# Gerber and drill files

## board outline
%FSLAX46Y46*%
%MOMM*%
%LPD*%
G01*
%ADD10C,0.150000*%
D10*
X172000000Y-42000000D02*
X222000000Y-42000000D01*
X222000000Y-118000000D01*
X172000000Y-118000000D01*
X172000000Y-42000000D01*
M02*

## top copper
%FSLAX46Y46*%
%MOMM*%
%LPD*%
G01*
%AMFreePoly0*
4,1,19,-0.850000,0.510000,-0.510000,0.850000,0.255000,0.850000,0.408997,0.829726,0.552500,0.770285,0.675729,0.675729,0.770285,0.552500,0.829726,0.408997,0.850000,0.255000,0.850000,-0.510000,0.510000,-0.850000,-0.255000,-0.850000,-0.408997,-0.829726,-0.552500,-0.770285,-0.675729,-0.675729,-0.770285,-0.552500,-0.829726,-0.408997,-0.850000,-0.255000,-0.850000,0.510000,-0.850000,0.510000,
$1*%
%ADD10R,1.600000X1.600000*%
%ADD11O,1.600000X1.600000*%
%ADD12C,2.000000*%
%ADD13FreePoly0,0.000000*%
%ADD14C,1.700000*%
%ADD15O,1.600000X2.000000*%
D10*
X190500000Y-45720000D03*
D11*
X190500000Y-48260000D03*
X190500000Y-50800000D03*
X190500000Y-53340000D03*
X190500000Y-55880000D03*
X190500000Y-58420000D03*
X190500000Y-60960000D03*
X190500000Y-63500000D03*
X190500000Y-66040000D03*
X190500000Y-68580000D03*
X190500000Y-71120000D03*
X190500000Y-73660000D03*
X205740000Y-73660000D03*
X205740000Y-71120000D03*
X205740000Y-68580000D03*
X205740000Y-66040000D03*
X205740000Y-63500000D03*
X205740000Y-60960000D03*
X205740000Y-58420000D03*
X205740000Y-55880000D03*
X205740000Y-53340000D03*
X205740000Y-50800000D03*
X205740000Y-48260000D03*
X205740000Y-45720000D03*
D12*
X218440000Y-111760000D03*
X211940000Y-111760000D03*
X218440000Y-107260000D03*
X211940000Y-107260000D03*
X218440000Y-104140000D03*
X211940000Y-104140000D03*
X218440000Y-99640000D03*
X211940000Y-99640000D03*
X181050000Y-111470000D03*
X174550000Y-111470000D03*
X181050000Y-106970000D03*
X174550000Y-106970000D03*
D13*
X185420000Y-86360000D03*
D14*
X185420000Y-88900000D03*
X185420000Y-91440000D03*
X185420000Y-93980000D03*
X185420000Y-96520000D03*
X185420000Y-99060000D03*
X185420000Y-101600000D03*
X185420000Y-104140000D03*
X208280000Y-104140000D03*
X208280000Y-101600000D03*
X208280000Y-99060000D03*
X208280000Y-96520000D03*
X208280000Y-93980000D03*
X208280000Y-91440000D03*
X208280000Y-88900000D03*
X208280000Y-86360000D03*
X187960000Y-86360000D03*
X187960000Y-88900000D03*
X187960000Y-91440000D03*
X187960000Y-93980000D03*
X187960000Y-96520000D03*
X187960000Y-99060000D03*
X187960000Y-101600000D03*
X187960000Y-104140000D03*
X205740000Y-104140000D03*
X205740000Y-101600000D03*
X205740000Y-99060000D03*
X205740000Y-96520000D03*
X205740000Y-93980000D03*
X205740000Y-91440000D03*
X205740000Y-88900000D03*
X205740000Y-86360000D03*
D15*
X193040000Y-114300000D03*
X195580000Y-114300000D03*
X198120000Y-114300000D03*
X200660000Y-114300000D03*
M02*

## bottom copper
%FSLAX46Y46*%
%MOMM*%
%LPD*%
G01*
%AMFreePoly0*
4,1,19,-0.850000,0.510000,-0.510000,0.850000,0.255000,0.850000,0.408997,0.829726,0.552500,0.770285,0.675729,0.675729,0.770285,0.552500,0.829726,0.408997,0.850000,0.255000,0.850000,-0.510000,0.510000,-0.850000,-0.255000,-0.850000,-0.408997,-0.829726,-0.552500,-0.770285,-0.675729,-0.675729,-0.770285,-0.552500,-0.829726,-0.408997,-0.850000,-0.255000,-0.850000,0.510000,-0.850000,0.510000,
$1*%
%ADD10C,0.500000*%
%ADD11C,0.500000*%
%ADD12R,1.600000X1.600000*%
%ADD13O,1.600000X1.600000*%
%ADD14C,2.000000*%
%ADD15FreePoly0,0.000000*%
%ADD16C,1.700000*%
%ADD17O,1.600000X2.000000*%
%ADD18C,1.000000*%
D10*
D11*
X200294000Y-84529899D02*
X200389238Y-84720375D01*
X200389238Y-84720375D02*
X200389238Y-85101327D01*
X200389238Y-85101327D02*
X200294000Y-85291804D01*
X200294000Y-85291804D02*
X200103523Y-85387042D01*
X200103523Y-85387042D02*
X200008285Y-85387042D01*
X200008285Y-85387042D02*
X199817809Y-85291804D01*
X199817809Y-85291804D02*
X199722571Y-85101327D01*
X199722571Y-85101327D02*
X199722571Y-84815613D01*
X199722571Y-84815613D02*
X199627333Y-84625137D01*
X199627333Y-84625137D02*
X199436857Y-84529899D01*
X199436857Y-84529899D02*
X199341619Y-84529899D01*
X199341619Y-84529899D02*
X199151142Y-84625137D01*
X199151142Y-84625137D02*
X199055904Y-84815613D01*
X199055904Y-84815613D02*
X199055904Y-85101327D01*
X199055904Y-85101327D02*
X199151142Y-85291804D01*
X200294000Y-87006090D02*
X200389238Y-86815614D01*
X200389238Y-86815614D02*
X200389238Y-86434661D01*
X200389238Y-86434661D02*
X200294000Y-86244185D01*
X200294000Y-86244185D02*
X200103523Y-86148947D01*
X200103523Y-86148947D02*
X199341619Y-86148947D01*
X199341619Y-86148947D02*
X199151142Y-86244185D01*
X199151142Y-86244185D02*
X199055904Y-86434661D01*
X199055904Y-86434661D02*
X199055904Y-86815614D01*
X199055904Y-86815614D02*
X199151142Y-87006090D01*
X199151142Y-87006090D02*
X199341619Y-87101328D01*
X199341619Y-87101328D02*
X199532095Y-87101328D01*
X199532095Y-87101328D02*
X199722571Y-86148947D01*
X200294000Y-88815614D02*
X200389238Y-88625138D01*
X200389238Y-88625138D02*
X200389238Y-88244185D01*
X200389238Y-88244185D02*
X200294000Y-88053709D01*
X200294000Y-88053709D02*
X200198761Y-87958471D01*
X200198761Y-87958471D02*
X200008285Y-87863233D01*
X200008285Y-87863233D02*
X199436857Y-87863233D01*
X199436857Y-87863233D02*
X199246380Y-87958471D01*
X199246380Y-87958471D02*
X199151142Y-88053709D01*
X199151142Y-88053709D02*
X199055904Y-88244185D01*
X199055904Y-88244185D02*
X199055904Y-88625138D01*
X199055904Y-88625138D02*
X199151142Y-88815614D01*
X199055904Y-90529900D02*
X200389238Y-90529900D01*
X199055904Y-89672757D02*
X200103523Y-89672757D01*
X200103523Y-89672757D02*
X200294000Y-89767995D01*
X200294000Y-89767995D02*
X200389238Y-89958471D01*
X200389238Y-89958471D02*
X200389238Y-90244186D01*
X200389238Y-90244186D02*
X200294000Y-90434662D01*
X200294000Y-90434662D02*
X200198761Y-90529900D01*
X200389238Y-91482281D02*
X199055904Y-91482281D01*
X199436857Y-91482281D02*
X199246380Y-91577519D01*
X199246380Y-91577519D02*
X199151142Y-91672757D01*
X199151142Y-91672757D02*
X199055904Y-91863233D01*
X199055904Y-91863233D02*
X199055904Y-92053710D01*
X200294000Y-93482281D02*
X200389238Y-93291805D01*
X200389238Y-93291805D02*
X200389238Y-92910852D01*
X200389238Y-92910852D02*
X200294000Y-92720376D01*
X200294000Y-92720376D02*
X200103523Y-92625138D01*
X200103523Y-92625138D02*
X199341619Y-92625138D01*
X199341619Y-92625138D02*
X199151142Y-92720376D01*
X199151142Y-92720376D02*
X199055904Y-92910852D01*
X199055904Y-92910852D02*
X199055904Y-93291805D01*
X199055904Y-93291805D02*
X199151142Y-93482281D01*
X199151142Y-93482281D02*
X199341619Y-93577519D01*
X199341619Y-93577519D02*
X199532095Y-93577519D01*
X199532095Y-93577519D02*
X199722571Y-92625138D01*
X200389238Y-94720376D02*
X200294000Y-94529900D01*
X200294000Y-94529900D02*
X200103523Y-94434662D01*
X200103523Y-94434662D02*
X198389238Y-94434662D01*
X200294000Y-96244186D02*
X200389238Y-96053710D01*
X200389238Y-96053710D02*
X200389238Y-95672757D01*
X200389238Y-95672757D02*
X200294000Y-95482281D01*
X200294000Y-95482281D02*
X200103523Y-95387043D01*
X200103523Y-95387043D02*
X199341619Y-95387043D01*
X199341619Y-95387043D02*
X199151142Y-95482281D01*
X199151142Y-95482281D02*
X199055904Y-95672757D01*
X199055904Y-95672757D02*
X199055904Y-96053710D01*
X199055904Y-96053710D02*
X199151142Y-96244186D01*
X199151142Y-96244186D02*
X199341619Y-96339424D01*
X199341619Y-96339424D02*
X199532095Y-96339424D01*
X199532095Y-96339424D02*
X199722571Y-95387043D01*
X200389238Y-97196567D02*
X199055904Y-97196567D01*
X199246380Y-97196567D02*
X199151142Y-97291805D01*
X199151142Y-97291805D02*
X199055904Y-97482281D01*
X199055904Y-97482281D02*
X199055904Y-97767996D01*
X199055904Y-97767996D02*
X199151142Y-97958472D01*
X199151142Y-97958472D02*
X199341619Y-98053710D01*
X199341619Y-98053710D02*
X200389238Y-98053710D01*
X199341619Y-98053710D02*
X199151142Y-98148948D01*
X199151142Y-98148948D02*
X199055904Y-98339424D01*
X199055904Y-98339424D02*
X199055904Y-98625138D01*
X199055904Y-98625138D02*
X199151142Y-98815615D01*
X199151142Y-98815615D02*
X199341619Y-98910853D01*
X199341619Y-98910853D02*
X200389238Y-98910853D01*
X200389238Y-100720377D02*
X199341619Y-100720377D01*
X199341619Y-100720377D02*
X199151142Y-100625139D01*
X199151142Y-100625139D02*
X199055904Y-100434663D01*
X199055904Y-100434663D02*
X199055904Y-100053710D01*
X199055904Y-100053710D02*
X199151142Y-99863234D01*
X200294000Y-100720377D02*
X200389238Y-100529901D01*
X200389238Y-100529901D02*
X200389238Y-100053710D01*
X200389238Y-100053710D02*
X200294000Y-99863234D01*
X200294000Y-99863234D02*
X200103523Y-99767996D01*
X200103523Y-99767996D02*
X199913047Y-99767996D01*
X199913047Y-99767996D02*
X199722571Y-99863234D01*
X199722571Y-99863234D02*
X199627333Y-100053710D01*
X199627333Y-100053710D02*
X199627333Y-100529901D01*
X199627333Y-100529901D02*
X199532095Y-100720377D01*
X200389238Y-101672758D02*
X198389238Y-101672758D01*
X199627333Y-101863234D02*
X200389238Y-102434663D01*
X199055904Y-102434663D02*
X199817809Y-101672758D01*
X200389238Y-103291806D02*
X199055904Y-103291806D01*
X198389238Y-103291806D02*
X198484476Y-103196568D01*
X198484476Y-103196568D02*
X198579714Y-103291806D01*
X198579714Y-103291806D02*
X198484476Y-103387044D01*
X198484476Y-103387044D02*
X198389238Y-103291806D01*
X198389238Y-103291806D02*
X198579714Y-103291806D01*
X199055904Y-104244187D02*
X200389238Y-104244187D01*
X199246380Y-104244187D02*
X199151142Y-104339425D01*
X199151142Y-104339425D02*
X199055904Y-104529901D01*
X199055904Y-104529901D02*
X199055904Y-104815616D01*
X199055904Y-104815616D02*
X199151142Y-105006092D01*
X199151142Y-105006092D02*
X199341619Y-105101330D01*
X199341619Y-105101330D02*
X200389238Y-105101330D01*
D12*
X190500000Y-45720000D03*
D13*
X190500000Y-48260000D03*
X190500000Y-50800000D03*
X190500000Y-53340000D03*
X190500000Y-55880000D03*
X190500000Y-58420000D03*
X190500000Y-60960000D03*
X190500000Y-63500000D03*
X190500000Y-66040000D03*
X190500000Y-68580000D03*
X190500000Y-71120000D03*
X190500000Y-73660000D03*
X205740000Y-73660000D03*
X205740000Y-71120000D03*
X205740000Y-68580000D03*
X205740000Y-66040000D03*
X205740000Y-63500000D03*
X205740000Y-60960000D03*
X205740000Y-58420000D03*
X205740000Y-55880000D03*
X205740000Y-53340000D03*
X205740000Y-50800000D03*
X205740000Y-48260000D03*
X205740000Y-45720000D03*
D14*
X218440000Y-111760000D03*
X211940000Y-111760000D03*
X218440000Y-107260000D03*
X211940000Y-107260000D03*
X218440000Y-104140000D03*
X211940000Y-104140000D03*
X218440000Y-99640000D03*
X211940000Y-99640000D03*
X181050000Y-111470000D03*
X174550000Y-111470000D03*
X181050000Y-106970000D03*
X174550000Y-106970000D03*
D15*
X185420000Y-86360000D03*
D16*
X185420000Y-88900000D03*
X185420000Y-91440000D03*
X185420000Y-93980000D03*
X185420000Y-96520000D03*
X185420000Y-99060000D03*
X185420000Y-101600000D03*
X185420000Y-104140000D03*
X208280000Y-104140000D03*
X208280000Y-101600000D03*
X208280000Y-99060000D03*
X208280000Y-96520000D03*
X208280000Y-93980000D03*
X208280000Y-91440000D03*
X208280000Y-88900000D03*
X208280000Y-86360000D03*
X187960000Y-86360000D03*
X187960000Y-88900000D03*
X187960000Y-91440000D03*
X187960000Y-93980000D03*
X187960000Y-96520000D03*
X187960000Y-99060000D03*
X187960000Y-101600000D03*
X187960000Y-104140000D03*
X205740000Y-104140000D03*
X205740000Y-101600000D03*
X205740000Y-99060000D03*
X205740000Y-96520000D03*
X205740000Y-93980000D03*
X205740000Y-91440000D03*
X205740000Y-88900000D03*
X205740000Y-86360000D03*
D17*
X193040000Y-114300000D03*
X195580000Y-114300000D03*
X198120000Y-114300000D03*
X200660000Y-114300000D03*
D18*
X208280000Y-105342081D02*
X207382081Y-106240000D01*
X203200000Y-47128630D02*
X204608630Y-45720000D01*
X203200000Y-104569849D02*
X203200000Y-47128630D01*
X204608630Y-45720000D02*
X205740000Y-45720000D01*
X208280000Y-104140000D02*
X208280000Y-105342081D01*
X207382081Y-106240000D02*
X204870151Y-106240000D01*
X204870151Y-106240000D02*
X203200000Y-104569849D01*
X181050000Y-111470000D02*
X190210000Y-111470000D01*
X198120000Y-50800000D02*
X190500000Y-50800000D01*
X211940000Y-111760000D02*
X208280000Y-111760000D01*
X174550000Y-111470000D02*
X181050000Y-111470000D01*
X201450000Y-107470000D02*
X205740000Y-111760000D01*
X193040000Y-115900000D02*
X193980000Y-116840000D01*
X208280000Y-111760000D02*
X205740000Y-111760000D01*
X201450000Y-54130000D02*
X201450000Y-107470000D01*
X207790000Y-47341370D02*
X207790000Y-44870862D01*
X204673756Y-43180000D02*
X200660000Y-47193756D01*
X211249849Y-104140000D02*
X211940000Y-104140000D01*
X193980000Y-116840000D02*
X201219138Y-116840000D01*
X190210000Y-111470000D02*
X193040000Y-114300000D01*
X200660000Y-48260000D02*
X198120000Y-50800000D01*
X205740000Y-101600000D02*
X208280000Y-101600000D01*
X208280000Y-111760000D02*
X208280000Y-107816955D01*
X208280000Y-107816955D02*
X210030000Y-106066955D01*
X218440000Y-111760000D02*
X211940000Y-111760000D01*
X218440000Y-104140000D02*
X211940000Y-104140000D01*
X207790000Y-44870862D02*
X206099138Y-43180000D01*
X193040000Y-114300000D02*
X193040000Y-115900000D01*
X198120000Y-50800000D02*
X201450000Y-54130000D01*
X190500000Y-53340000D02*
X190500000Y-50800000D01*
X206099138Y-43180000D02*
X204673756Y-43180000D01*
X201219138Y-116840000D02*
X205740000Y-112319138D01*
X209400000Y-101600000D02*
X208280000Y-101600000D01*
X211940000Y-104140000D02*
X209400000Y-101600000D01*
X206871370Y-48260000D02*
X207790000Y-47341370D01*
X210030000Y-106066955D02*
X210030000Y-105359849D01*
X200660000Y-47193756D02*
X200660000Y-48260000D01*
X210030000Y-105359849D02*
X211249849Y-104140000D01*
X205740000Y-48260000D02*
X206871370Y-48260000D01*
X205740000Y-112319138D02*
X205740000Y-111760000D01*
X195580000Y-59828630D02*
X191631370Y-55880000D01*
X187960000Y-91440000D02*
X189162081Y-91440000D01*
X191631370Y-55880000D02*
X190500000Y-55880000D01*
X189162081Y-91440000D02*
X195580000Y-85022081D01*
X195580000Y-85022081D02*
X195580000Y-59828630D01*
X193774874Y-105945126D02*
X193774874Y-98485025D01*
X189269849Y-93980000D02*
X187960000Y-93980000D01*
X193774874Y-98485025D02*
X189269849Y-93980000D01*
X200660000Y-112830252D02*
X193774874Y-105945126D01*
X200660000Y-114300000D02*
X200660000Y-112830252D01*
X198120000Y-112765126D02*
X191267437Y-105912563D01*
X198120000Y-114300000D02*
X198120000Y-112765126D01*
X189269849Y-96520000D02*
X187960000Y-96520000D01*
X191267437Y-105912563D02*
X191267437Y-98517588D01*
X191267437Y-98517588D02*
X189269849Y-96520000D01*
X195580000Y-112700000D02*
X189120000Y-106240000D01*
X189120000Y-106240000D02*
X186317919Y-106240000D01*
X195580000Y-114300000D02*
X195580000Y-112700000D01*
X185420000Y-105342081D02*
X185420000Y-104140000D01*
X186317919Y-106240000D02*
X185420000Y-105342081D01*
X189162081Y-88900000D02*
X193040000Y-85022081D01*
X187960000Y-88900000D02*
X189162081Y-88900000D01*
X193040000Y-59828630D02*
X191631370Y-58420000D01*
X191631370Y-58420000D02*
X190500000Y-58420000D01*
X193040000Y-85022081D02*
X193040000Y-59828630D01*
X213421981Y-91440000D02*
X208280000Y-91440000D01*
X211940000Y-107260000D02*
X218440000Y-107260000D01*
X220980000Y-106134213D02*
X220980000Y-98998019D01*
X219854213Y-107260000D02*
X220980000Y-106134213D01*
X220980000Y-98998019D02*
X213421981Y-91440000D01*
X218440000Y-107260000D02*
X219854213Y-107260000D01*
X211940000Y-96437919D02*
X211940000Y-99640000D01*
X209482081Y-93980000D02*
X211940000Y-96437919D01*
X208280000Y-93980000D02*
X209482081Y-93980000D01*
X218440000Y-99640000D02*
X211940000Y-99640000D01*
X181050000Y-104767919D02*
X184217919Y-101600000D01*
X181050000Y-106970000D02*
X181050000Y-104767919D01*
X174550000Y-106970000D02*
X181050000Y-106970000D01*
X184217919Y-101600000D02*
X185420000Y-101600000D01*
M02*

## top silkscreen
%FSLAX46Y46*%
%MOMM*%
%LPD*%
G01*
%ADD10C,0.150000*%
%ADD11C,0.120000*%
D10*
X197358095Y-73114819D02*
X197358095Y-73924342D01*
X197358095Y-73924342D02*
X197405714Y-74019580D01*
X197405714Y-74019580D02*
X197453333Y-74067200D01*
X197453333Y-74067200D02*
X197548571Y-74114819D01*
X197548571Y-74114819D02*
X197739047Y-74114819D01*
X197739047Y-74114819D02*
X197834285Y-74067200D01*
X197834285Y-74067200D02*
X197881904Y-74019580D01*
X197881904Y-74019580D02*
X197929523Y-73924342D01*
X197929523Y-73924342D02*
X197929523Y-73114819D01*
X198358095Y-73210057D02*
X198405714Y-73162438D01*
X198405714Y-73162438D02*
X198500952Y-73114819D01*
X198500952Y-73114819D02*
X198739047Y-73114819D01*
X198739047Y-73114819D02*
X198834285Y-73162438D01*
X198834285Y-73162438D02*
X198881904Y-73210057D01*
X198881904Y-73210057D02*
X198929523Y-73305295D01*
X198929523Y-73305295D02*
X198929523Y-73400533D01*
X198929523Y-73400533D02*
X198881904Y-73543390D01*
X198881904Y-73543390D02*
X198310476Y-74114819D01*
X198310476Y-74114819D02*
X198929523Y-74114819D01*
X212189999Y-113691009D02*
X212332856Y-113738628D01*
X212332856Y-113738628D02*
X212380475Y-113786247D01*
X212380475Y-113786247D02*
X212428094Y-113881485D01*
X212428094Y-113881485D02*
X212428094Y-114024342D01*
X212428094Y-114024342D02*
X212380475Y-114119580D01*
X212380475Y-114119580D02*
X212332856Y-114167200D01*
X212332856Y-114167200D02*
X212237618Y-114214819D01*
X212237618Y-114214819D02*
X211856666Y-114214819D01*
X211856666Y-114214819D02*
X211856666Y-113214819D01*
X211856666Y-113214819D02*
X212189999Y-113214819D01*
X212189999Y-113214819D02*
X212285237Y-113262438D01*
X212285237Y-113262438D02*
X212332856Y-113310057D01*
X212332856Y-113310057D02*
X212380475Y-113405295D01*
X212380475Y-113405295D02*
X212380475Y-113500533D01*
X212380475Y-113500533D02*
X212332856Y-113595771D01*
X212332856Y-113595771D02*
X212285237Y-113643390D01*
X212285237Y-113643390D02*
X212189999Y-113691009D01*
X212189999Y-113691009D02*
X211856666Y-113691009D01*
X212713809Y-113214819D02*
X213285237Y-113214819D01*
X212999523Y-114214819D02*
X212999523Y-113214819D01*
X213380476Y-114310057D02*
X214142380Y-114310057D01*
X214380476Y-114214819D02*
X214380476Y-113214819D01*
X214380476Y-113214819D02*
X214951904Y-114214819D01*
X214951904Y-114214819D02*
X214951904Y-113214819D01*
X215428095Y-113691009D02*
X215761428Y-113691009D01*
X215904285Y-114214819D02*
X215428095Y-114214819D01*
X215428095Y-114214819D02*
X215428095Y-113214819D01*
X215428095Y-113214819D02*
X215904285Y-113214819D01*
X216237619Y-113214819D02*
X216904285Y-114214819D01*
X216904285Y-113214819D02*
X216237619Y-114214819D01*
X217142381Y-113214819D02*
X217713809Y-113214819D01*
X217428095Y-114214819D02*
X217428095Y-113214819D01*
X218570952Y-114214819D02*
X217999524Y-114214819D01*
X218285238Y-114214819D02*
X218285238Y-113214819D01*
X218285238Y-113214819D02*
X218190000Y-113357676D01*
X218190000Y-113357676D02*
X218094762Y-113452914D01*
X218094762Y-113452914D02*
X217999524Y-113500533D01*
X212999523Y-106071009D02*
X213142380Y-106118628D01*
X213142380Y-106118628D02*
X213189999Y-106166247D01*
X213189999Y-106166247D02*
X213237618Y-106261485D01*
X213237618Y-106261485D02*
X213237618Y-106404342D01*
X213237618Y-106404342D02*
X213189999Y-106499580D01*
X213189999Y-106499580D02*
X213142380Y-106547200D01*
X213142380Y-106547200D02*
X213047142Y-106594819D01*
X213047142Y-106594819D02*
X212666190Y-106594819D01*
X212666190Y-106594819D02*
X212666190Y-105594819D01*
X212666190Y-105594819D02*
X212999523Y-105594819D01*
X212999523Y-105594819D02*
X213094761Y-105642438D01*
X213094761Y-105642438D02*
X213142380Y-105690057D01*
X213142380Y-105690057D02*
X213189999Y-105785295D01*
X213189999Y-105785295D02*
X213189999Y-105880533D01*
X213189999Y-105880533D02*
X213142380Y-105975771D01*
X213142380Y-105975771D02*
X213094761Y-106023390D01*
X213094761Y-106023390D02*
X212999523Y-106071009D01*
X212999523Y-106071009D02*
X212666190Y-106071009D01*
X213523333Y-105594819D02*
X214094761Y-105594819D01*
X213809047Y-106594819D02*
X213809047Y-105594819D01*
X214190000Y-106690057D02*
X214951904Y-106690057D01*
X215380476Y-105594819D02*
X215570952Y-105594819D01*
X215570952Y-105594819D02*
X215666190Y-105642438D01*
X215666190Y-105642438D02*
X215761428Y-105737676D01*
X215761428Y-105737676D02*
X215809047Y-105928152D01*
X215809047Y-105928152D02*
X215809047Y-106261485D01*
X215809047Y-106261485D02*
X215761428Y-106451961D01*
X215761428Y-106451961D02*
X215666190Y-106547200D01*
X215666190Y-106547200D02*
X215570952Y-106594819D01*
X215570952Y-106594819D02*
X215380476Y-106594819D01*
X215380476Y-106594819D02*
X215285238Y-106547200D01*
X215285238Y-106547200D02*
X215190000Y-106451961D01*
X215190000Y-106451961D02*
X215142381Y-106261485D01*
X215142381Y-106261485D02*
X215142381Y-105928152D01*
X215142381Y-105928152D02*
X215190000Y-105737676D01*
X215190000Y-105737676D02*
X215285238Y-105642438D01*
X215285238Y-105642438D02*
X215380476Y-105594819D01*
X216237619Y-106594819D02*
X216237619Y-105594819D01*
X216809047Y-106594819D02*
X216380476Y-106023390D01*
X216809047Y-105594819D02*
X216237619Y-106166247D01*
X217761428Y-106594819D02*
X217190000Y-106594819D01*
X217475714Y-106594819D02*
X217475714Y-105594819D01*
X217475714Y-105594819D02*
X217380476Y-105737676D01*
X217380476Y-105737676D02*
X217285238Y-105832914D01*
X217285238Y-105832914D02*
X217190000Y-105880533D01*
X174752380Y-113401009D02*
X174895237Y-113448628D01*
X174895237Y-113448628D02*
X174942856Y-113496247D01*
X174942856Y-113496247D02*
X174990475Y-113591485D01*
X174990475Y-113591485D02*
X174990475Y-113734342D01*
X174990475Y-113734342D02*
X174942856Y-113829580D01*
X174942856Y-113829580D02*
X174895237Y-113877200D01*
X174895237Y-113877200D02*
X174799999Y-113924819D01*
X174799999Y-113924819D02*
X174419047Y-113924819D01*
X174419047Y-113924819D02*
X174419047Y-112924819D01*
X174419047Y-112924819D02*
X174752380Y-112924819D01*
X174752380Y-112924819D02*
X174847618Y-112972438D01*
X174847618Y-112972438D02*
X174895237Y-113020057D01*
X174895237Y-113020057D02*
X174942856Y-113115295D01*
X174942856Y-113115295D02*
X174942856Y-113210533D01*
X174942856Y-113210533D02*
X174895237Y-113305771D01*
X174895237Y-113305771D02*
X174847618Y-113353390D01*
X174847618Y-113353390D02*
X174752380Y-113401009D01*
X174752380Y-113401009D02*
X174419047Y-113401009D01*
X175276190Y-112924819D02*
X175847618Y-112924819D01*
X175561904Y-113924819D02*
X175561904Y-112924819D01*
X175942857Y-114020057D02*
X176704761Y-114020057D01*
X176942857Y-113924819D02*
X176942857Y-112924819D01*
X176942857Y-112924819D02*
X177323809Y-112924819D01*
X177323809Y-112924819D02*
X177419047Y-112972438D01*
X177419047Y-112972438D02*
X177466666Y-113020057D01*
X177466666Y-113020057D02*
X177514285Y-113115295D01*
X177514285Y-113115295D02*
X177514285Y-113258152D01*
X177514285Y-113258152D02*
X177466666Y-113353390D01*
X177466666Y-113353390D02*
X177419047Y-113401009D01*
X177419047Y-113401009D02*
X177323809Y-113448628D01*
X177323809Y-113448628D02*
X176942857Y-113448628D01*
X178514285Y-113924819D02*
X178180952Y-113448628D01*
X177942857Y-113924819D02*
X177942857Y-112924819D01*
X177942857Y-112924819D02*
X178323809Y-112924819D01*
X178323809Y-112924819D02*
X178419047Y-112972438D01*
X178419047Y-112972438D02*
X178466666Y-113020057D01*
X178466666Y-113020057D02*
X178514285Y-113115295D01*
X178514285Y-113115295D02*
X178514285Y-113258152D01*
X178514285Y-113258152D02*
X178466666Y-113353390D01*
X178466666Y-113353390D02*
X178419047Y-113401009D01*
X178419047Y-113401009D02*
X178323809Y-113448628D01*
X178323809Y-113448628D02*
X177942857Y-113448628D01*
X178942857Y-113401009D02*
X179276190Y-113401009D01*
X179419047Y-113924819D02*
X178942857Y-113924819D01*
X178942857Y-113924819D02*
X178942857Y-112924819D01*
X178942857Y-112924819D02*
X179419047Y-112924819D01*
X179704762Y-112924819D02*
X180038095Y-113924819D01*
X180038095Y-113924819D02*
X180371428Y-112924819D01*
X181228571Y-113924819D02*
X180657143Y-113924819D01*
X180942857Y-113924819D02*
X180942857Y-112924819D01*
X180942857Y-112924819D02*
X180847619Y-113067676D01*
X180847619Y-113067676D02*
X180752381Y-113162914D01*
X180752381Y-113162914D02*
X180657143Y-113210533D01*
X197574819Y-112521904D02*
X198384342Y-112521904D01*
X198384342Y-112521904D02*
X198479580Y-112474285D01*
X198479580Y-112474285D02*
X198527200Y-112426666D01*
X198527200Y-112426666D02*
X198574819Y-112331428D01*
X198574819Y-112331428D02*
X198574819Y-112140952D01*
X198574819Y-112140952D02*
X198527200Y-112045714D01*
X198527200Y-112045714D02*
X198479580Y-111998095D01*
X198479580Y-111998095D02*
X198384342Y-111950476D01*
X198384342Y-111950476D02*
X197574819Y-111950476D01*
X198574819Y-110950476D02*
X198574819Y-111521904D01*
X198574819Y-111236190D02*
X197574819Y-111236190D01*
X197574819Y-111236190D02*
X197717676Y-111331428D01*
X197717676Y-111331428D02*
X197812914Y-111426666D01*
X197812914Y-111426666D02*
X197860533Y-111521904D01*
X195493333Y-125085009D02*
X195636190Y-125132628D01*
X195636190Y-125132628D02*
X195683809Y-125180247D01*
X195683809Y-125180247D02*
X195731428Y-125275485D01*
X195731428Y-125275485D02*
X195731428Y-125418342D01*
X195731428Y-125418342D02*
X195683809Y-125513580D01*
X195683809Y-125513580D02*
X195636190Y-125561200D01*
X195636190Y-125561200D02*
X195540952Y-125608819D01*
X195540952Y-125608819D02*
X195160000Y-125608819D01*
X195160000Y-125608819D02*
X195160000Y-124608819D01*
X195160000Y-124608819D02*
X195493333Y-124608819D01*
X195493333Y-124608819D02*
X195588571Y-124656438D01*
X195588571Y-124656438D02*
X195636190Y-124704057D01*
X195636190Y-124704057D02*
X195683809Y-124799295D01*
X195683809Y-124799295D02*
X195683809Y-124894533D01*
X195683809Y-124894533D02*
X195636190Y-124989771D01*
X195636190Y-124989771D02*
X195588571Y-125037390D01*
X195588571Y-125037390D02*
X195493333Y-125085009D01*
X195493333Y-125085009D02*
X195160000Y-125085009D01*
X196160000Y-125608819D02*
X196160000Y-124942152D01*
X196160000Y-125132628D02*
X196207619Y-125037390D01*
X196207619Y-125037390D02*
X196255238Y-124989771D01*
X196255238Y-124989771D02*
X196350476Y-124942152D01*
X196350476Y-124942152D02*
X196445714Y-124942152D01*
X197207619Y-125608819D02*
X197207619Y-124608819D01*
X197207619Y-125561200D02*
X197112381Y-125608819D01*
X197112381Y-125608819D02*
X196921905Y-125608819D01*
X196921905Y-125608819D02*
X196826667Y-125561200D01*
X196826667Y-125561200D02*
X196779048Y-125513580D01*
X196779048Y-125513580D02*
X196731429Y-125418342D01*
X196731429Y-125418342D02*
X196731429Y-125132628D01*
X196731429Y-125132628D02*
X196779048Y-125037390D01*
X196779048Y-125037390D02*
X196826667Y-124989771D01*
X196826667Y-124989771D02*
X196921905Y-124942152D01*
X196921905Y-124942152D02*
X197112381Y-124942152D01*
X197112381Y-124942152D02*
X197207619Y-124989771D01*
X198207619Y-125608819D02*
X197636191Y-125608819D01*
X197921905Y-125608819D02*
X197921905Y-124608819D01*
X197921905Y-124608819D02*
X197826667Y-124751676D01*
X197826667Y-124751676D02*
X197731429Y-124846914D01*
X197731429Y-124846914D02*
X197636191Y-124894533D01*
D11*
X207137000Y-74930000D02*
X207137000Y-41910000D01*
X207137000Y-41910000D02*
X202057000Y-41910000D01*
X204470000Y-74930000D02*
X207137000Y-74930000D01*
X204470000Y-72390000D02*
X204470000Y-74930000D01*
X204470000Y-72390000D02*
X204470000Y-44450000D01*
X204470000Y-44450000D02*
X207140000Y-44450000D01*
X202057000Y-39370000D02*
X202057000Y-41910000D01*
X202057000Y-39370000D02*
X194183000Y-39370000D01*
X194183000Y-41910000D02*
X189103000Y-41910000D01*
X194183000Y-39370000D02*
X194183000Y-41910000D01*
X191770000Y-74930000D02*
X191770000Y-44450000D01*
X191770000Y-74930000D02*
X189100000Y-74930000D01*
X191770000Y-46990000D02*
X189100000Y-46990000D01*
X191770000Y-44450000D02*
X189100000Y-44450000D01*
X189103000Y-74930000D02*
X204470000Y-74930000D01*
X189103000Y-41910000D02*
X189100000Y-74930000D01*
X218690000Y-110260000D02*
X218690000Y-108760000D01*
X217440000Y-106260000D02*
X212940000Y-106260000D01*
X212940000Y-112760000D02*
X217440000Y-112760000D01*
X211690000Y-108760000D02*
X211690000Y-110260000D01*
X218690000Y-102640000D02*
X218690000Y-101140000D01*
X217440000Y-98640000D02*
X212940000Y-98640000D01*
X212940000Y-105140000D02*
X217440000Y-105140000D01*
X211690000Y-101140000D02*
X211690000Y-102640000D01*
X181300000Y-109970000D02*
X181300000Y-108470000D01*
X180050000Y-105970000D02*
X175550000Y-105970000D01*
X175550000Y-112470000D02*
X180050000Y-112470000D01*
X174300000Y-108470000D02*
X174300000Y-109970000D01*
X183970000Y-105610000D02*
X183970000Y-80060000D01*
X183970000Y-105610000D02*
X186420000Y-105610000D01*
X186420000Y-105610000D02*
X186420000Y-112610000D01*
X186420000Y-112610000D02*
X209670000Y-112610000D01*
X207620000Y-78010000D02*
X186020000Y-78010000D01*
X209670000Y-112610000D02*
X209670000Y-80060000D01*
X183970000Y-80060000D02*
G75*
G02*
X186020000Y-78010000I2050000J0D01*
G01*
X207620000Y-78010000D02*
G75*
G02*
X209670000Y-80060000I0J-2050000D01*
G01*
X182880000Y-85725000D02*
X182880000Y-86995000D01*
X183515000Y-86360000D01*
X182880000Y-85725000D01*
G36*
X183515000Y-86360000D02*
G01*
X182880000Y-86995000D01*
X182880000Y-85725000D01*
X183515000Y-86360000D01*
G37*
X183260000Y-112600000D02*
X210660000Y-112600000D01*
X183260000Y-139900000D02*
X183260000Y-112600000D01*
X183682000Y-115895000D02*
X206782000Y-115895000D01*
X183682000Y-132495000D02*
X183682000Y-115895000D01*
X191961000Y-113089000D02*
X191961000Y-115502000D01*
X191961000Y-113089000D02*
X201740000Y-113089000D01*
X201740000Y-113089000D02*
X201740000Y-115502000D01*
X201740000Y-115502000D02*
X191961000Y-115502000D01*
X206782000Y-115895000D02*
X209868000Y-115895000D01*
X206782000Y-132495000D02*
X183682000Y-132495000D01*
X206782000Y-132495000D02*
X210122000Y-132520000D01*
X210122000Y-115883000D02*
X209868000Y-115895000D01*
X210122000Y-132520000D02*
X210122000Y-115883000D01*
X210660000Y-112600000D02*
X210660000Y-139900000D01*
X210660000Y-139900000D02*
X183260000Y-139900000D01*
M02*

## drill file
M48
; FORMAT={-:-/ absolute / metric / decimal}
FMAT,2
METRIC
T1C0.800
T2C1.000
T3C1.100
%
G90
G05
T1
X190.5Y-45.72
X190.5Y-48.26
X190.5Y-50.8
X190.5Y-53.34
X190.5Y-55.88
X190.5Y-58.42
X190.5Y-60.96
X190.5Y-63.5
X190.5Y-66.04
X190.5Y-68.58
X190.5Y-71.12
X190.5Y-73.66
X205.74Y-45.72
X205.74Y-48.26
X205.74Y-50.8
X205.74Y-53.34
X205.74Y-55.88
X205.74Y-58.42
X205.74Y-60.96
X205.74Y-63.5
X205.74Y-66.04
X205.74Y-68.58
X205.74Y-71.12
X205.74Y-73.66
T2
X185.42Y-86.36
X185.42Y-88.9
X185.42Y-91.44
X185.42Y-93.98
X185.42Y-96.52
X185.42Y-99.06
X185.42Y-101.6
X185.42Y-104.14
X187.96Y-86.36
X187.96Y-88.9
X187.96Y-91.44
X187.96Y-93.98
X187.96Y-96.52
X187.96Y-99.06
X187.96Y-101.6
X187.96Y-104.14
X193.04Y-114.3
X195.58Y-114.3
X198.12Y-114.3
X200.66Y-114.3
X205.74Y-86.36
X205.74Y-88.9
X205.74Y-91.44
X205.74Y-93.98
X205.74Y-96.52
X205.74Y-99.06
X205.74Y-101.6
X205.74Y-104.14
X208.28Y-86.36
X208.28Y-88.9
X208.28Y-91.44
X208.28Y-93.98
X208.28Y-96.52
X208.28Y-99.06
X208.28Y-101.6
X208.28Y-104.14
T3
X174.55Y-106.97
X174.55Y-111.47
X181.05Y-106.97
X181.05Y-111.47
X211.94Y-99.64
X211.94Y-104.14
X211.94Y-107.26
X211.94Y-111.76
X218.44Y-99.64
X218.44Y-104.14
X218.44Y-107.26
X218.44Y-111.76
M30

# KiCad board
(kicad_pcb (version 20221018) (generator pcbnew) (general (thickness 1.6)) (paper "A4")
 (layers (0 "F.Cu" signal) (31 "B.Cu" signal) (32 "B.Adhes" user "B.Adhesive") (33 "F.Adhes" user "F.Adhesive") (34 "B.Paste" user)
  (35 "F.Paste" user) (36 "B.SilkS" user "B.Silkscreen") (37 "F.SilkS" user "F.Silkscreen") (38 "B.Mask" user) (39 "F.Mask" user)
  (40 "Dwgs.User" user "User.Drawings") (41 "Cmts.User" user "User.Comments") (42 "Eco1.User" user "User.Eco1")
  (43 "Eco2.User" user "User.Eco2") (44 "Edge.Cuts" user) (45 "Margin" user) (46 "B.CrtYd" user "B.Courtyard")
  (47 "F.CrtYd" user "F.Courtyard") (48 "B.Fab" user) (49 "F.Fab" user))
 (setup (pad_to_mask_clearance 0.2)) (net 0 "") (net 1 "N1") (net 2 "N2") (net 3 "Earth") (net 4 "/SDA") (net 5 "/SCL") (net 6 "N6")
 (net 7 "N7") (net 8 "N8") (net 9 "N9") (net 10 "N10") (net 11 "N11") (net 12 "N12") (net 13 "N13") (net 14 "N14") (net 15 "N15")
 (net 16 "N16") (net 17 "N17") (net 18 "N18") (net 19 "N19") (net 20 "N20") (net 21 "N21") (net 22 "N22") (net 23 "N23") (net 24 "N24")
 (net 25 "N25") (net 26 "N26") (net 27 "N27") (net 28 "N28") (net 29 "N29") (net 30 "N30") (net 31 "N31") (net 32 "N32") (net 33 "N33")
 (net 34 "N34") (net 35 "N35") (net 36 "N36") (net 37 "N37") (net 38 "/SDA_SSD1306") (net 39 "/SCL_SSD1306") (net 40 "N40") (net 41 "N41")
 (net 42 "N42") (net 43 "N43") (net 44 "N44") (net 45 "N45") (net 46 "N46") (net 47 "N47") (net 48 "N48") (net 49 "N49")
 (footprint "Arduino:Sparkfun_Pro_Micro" (layer "F.Cu") (at 205.74 73.66 180)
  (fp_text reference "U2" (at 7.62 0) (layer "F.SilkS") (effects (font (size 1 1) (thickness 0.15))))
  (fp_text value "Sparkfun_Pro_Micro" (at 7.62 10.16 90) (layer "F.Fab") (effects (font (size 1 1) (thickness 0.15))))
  (fp_line (start -1.397 -1.27) (end -1.397 31.75) (stroke (width 0.12) (type solid)) (layer "F.SilkS"))
  (fp_line (start -1.397 31.75) (end 3.683 31.75) (stroke (width 0.12) (type solid)) (layer "F.SilkS"))
  (fp_line (start 1.27 -1.27) (end -1.397 -1.27) (stroke (width 0.12) (type solid)) (layer "F.SilkS"))
  (fp_line (start 1.27 1.27) (end 1.27 -1.27) (stroke (width 0.12) (type solid)) (layer "F.SilkS"))
  (fp_line (start 1.27 1.27) (end 1.27 29.21) (stroke (width 0.12) (type solid)) (layer "F.SilkS"))
  (fp_line (start 1.27 29.21) (end -1.4 29.21) (stroke (width 0.12) (type solid)) (layer "F.SilkS"))
  (fp_line (start 3.683 34.29) (end 3.683 31.75) (stroke (width 0.12) (type solid)) (layer "F.SilkS"))
  (fp_line (start 3.683 34.29) (end 11.557 34.29) (stroke (width 0.12) (type solid)) (layer "F.SilkS"))
  (fp_line (start 11.557 31.75) (end 16.637 31.75) (stroke (width 0.12) (type solid)) (layer "F.SilkS"))
  (fp_line (start 11.557 34.29) (end 11.557 31.75) (stroke (width 0.12) (type solid)) (layer "F.SilkS"))
  (fp_line (start 13.97 -1.27) (end 13.97 29.21) (stroke (width 0.12) (type solid)) (layer "F.SilkS"))
  (fp_line (start 13.97 -1.27) (end 16.64 -1.27) (stroke (width 0.12) (type solid)) (layer "F.SilkS"))
  (fp_line (start 13.97 26.67) (end 16.64 26.67) (stroke (width 0.12) (type solid)) (layer "F.SilkS"))
  (fp_line (start 13.97 29.21) (end 16.64 29.21) (stroke (width 0.12) (type solid)) (layer "F.SilkS"))
  (fp_line (start 16.637 -1.27) (end 1.27 -1.27) (stroke (width 0.12) (type solid)) (layer "F.SilkS"))
  (fp_line (start 16.637 31.75) (end 16.64 -1.27) (stroke (width 0.12) (type solid)) (layer "F.SilkS"))
  (pad "1" thru_hole rect (at 15.24 27.94 180) (size 1.6 1.6) (drill 0.8) (layers "*.Cu" "*.Mask") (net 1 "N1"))
  (pad "2" thru_hole oval (at 15.24 25.4 180) (size 1.6 1.6) (drill 0.8) (layers "*.Cu" "*.Mask") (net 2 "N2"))
  (pad "3" thru_hole oval (at 15.24 22.86 180) (size 1.6 1.6) (drill 0.8) (layers "*.Cu" "*.Mask") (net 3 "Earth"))
  (pad "4" thru_hole oval (at 15.24 20.32 180) (size 1.6 1.6) (drill 0.8) (layers "*.Cu" "*.Mask") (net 3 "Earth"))
  (pad "5" thru_hole oval (at 15.24 17.78 180) (size 1.6 1.6) (drill 0.8) (layers "*.Cu" "*.Mask") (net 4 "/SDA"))
  (pad "6" thru_hole oval (at 15.24 15.24 180) (size 1.6 1.6) (drill 0.8) (layers "*.Cu" "*.Mask") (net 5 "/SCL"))
  (pad "7" thru_hole oval (at 15.24 12.7 180) (size 1.6 1.6) (drill 0.8) (layers "*.Cu" "*.Mask") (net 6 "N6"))
  (pad "8" thru_hole oval (at 15.24 10.16 180) (size 1.6 1.6) (drill 0.8) (layers "*.Cu" "*.Mask") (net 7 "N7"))
  (pad "9" thru_hole oval (at 15.24 7.62 180) (size 1.6 1.6) (drill 0.8) (layers "*.Cu" "*.Mask") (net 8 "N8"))
  (pad "10" thru_hole oval (at 15.24 5.08 180) (size 1.6 1.6) (drill 0.8) (layers "*.Cu" "*.Mask") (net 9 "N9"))
  (pad "11" thru_hole oval (at 15.24 2.54 180) (size 1.6 1.6) (drill 0.8) (layers "*.Cu" "*.Mask") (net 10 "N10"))
  (pad "12" thru_hole oval (at 15.24 0 180) (size 1.6 1.6) (drill 0.8) (layers "*.Cu" "*.Mask") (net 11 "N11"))
  (pad "13" thru_hole oval (at 0 0 180) (size 1.6 1.6) (drill 0.8) (layers "*.Cu" "*.Mask") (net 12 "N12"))
  (pad "14" thru_hole oval (at 0 2.54 180) (size 1.6 1.6) (drill 0.8) (layers "*.Cu" "*.Mask") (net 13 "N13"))
  (pad "15" thru_hole oval (at 0 5.08 180) (size 1.6 1.6) (drill 0.8) (layers "*.Cu" "*.Mask") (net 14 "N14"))
  (pad "16" thru_hole oval (at 0 7.62 180) (size 1.6 1.6) (drill 0.8) (layers "*.Cu" "*.Mask") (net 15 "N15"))
  (pad "17" thru_hole oval (at 0 10.16 180) (size 1.6 1.6) (drill 0.8) (layers "*.Cu" "*.Mask") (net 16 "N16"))
  (pad "18" thru_hole oval (at 0 12.7 180) (size 1.6 1.6) (drill 0.8) (layers "*.Cu" "*.Mask") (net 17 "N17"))
  (pad "19" thru_hole oval (at 0 15.24 180) (size 1.6 1.6) (drill 0.8) (layers "*.Cu" "*.Mask") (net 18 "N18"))
  (pad "20" thru_hole oval (at 0 17.78 180) (size 1.6 1.6) (drill 0.8) (layers "*.Cu" "*.Mask") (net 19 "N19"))
  (pad "21" thru_hole oval (at 0 20.32 180) (size 1.6 1.6) (drill 0.8) (layers "*.Cu" "*.Mask") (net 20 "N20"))
  (pad "22" thru_hole oval (at 0 22.86 180) (size 1.6 1.6) (drill 0.8) (layers "*.Cu" "*.Mask") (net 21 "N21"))
  (pad "23" thru_hole oval (at 0 25.4 180) (size 1.6 1.6) (drill 0.8) (layers "*.Cu" "*.Mask") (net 3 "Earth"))
  (pad "24" thru_hole oval (at 0 27.94 180) (size 1.6 1.6) (drill 0.8) (layers "*.Cu" "*.Mask") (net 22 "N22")))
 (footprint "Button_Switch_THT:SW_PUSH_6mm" (layer "F.Cu") (at 218.44 111.76 180)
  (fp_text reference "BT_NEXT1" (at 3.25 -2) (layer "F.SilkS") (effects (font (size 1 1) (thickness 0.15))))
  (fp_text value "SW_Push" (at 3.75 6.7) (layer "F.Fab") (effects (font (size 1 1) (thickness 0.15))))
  (fp_line (start -0.25 1.5) (end -0.25 3) (stroke (width 0.12) (type solid)) (layer "F.SilkS"))
  (fp_line (start 1 5.5) (end 5.5 5.5) (stroke (width 0.12) (type solid)) (layer "F.SilkS"))
  (fp_line (start 5.5 -1) (end 1 -1) (stroke (width 0.12) (type solid)) (layer "F.SilkS"))
  (fp_line (start 6.75 3) (end 6.75 1.5) (stroke (width 0.12) (type solid)) (layer "F.SilkS"))
  (pad "1" thru_hole circle (at 0 0 270) (size 2 2) (drill 1.1) (layers "*.Cu" "*.Mask") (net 3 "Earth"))
  (pad "1" thru_hole circle (at 6.5 0 270) (size 2 2) (drill 1.1) (layers "*.Cu" "*.Mask") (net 3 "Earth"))
  (pad "2" thru_hole circle (at 0 4.5 270) (size 2 2) (drill 1.1) (layers "*.Cu" "*.Mask") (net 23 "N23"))
  (pad "2" thru_hole circle (at 6.5 4.5 270) (size 2 2) (drill 1.1) (layers "*.Cu" "*.Mask") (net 23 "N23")))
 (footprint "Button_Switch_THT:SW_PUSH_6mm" (layer "F.Cu") (at 218.44 104.14 180)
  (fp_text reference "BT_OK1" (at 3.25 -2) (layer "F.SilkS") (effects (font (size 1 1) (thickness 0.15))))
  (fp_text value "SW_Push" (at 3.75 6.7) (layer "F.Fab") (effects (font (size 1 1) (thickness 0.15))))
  (fp_line (start -0.25 1.5) (end -0.25 3) (stroke (width 0.12) (type solid)) (layer "F.SilkS"))
  (fp_line (start 1 5.5) (end 5.5 5.5) (stroke (width 0.12) (type solid)) (layer "F.SilkS"))
  (fp_line (start 5.5 -1) (end 1 -1) (stroke (width 0.12) (type solid)) (layer "F.SilkS"))
  (fp_line (start 6.75 3) (end 6.75 1.5) (stroke (width 0.12) (type solid)) (layer "F.SilkS"))
  (pad "1" thru_hole circle (at 0 0 270) (size 2 2) (drill 1.1) (layers "*.Cu" "*.Mask") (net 3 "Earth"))
  (pad "1" thru_hole circle (at 6.5 0 270) (size 2 2) (drill 1.1) (layers "*.Cu" "*.Mask") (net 3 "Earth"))
  (pad "2" thru_hole circle (at 0 4.5 270) (size 2 2) (drill 1.1) (layers "*.Cu" "*.Mask") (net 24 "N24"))
  (pad "2" thru_hole circle (at 6.5 4.5 270) (size 2 2) (drill 1.1) (layers "*.Cu" "*.Mask") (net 24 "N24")))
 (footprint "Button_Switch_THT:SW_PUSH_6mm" (layer "F.Cu") (at 181.05 111.47 180)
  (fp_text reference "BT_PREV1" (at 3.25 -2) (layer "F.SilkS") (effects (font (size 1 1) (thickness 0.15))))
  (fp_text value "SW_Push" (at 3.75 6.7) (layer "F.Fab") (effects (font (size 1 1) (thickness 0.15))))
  (fp_line (start -0.25 1.5) (end -0.25 3) (stroke (width 0.12) (type solid)) (layer "F.SilkS"))
  (fp_line (start 1 5.5) (end 5.5 5.5) (stroke (width 0.12) (type solid)) (layer "F.SilkS"))
  (fp_line (start 5.5 -1) (end 1 -1) (stroke (width 0.12) (type solid)) (layer "F.SilkS"))
  (fp_line (start 6.75 3) (end 6.75 1.5) (stroke (width 0.12) (type solid)) (layer "F.SilkS"))
  (pad "1" thru_hole circle (at 0 0 270) (size 2 2) (drill 1.1) (layers "*.Cu" "*.Mask") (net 3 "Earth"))
  (pad "1" thru_hole circle (at 6.5 0 270) (size 2 2) (drill 1.1) (layers "*.Cu" "*.Mask") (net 3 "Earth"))
  (pad "2" thru_hole circle (at 0 4.5 270) (size 2 2) (drill 1.1) (layers "*.Cu" "*.Mask") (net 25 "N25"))
  (pad "2" thru_hole circle (at 6.5 4.5 270) (size 2 2) (drill 1.1) (layers "*.Cu" "*.Mask") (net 25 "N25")))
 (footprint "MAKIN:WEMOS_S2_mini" (layer "F.Cu") (at 185.42 86.36)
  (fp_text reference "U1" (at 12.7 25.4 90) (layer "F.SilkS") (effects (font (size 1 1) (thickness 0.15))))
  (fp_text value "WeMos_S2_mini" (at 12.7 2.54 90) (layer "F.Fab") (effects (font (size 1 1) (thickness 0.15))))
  (fp_line (start -1.45 19.25) (end -1.45 -6.3) (stroke (width 0.12) (type solid)) (layer "F.SilkS"))
  (fp_line (start -1.45 19.25) (end 1 19.25) (stroke (width 0.12) (type solid)) (layer "F.SilkS"))
  (fp_line (start 1 19.25) (end 1 26.25) (stroke (width 0.12) (type solid)) (layer "F.SilkS"))
  (fp_line (start 1 26.25) (end 24.25 26.25) (stroke (width 0.12) (type solid)) (layer "F.SilkS"))
  (fp_line (start 22.2 -8.35) (end 0.6 -8.35) (stroke (width 0.12) (type solid)) (layer "F.SilkS"))
  (fp_line (start 24.25 26.25) (end 24.25 -6.3) (stroke (width 0.12) (type solid)) (layer "F.SilkS"))
  (fp_arc (start -1.45 -6.3) (mid -0.849569 -7.749569) (end 0.6 -8.35) (stroke (width 0.12) (type solid)) (layer "F.SilkS"))
  (fp_arc (start 22.2 -8.35) (mid 23.649569 -7.749569) (end 24.25 -6.3) (stroke (width 0.12) (type solid)) (layer "F.SilkS"))
  (fp_poly (pts (xy -2.54 -0.635) (xy -2.54 0.635) (xy -1.905 0)) (stroke (width 0.12) (type solid)) (fill solid) (layer "F.SilkS"))
  (pad "1" thru_hole roundrect (at 0 0) (size 1.7 1.7) (drill 1) (layers "*.Cu" "*.Mask") (roundrect_rratio 0.35) (chamfer_ratio 0.2)
   (chamfer top_left bottom_right) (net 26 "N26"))
  (pad "2" thru_hole circle (at 0 2.54) (size 1.7 1.7) (drill 1) (layers "*.Cu" "*.Mask") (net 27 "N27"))
  (pad "3" thru_hole circle (at 0 5.08) (size 1.7 1.7) (drill 1) (layers "*.Cu" "*.Mask") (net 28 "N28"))
  (pad "4" thru_hole circle (at 0 7.62) (size 1.7 1.7) (drill 1) (layers "*.Cu" "*.Mask") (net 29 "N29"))
  (pad "5" thru_hole circle (at 0 10.16) (size 1.7 1.7) (drill 1) (layers "*.Cu" "*.Mask") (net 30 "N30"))
  (pad "6" thru_hole circle (at 0 12.7) (size 1.7 1.7) (drill 1) (layers "*.Cu" "*.Mask") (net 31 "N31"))
  (pad "7" thru_hole circle (at 0 15.24) (size 1.7 1.7) (drill 1) (layers "*.Cu" "*.Mask") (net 25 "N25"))
  (pad "8" thru_hole circle (at 0 17.78) (size 1.7 1.7) (drill 1) (layers "*.Cu" "*.Mask") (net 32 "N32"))
  (pad "9" thru_hole circle (at 22.86 17.78) (size 1.7 1.7) (drill 1) (layers "*.Cu" "*.Mask") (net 22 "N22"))
  (pad "10" thru_hole circle (at 22.86 15.24) (size 1.7 1.7) (drill 1) (layers "*.Cu" "*.Mask") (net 3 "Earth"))
  (pad "11" thru_hole circle (at 22.86 12.7) (size 1.7 1.7) (drill 1) (layers "*.Cu" "*.Mask") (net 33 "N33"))
  (pad "12" thru_hole circle (at 22.86 10.16) (size 1.7 1.7) (drill 1) (layers "*.Cu" "*.Mask") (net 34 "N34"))
  (pad "13" thru_hole circle (at 22.86 7.62) (size 1.7 1.7) (drill 1) (layers "*.Cu" "*.Mask") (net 24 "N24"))
  (pad "14" thru_hole circle (at 22.86 5.08) (size 1.7 1.7) (drill 1) (layers "*.Cu" "*.Mask") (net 23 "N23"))
  (pad "15" thru_hole circle (at 22.86 2.54) (size 1.7 1.7) (drill 1) (layers "*.Cu" "*.Mask") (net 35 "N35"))
  (pad "16" thru_hole circle (at 22.86 0) (size 1.7 1.7) (drill 1) (layers "*.Cu" "*.Mask") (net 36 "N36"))
  (pad "17" thru_hole circle (at 2.54 0) (size 1.7 1.7) (drill 1) (layers "*.Cu" "*.Mask") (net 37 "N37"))
  (pad "18" thru_hole circle (at 2.54 2.54) (size 1.7 1.7) (drill 1) (layers "*.Cu" "*.Mask") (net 5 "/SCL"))
  (pad "19" thru_hole circle (at 2.54 5.08) (size 1.7 1.7) (drill 1) (layers "*.Cu" "*.Mask") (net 4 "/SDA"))
  (pad "20" thru_hole circle (at 2.54 7.62) (size 1.7 1.7) (drill 1) (layers "*.Cu" "*.Mask") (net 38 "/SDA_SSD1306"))
  (pad "21" thru_hole circle (at 2.54 10.16) (size 1.7 1.7) (drill 1) (layers "*.Cu" "*.Mask") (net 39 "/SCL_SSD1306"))
  (pad "22" thru_hole circle (at 2.54 12.7) (size 1.7 1.7) (drill 1) (layers "*.Cu" "*.Mask") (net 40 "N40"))
  (pad "23" thru_hole circle (at 2.54 15.24) (size 1.7 1.7) (drill 1) (layers "*.Cu" "*.Mask") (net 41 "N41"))
  (pad "24" thru_hole circle (at 2.54 17.78) (size 1.7 1.7) (drill 1) (layers "*.Cu" "*.Mask") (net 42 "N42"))
  (pad "25" thru_hole circle (at 20.32 17.78) (size 1.7 1.7) (drill 1) (layers "*.Cu" "*.Mask") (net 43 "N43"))
  (pad "26" thru_hole circle (at 20.32 15.24) (size 1.7 1.7) (drill 1) (layers "*.Cu" "*.Mask") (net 3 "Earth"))
  (pad "27" thru_hole circle (at 20.32 12.7) (size 1.7 1.7) (drill 1) (layers "*.Cu" "*.Mask") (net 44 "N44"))
  (pad "28" thru_hole circle (at 20.32 10.16) (size 1.7 1.7) (drill 1) (layers "*.Cu" "*.Mask") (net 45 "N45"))
  (pad "29" thru_hole circle (at 20.32 7.62) (size 1.7 1.7) (drill 1) (layers "*.Cu" "*.Mask") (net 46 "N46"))
  (pad "30" thru_hole circle (at 20.32 5.08) (size 1.7 1.7) (drill 1) (layers "*.Cu" "*.Mask") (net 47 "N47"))
  (pad "31" thru_hole circle (at 20.32 2.54) (size 1.7 1.7) (drill 1) (layers "*.Cu" "*.Mask") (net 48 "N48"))
  (pad "32" thru_hole circle (at 20.32 0) (size 1.7 1.7) (drill 1) (layers "*.Cu" "*.Mask") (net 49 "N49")))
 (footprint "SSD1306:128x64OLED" (layer "F.Cu") (at 196.66 124.9)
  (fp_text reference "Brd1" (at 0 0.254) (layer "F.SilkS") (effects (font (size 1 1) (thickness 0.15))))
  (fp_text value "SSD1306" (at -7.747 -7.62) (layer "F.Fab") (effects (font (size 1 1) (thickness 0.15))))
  (fp_line (start -13.4 -12.3) (end 14 -12.3) (stroke (width 0.12) (type solid)) (layer "F.SilkS"))
  (fp_line (start -13.4 15) (end -13.4 -12.3) (stroke (width 0.12) (type solid)) (layer "F.SilkS"))
  (fp_line (start -12.978 -9.005) (end 10.122 -9.005) (stroke (width 0.12) (type solid)) (layer "F.SilkS"))
  (fp_line (start -12.978 7.595) (end -12.978 -9.005) (stroke (width 0.12) (type solid)) (layer "F.SilkS"))
  (fp_line (start -4.699 -11.811) (end -4.699 -9.398) (stroke (width 0.12) (type solid)) (layer "F.SilkS"))
  (fp_line (start -4.699 -11.811) (end 5.08 -11.811) (stroke (width 0.12) (type solid)) (layer "F.SilkS"))
  (fp_line (start 5.08 -11.811) (end 5.08 -9.398) (stroke (width 0.12) (type solid)) (layer "F.SilkS"))
  (fp_line (start 5.08 -9.398) (end -4.699 -9.398) (stroke (width 0.12) (type solid)) (layer "F.SilkS"))
  (fp_line (start 10.122 -9.005) (end 13.208 -9.005) (stroke (width 0.12) (type solid)) (layer "F.SilkS"))
  (fp_line (start 10.122 7.595) (end -12.978 7.595) (stroke (width 0.12) (type solid)) (layer "F.SilkS"))
  (fp_line (start 10.122 7.595) (end 13.462 7.62) (stroke (width 0.12) (type solid)) (layer "F.SilkS"))
  (fp_line (start 13.462 -9.017) (end 13.208 -9.005) (stroke (width 0.12) (type solid)) (layer "F.SilkS"))
  (fp_line (start 13.462 7.62) (end 13.462 -9.017) (stroke (width 0.12) (type solid)) (layer "F.SilkS"))
  (fp_line (start 14 -12.3) (end 14 15) (stroke (width 0.12) (type solid)) (layer "F.SilkS"))
  (fp_line (start 14 15) (end -13.4 15) (stroke (width 0.12) (type solid)) (layer "F.SilkS"))
  (pad "1" thru_hole oval (at -3.62 -10.6 90) (size 2 1.6) (drill 1) (layers "*.Cu" "*.Mask") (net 3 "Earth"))
  (pad "2" thru_hole oval (at -1.08 -10.6 90) (size 2 1.6) (drill 1) (layers "*.Cu" "*.Mask") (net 32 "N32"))
  (pad "3" thru_hole oval (at 1.46 -10.6 90) (size 2 1.6) (drill 1) (layers "*.Cu" "*.Mask") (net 39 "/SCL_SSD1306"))
  (pad "4" thru_hole oval (at 4 -10.6 90) (size 2 1.6) (drill 1) (layers "*.Cu" "*.Mask") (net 38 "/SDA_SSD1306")))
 (gr_rect (start 172 42) (end 222 118) (stroke (width 0.15) (type default)) (fill none) (layer "Edge.Cuts"))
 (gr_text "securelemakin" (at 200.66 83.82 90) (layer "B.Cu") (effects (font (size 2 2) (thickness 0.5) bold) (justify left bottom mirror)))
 (segment (start 208.28 105.342081) (end 207.382081 106.24) (width 1) (layer "B.Cu") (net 22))
 (segment (start 203.2 47.12863) (end 204.60863 45.72) (width 1) (layer "B.Cu") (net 22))
 (segment (start 203.2 104.569849) (end 203.2 47.12863) (width 1) (layer "B.Cu") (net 22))
 (segment (start 204.60863 45.72) (end 205.74 45.72) (width 1) (layer "B.Cu") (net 22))
 (segment (start 208.28 104.14) (end 208.28 105.342081) (width 1) (layer "B.Cu") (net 22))
 (segment (start 207.382081 106.24) (end 204.870151 106.24) (width 1) (layer "B.Cu") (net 22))
 (segment (start 204.870151 106.24) (end 203.2 104.569849) (width 1) (layer "B.Cu") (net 22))
 (segment (start 181.05 111.47) (end 190.21 111.47) (width 1) (layer "B.Cu") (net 3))
 (segment (start 198.12 50.8) (end 190.5 50.8) (width 1) (layer "B.Cu") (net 3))
 (segment (start 211.94 111.76) (end 208.28 111.76) (width 1) (layer "B.Cu") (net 3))
 (segment (start 174.55 111.47) (end 181.05 111.47) (width 1) (layer "B.Cu") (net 3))
 (segment (start 201.45 107.47) (end 205.74 111.76) (width 1) (layer "B.Cu") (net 3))
 (segment (start 193.04 115.9) (end 193.98 116.84) (width 1) (layer "B.Cu") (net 3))
 (segment (start 208.28 111.76) (end 205.74 111.76) (width 1) (layer "B.Cu") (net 3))
 (segment (start 201.45 54.13) (end 201.45 107.47) (width 1) (layer "B.Cu") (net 3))
 (segment (start 207.79 47.34137) (end 207.79 44.870862) (width 1) (layer "B.Cu") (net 3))
 (segment (start 204.673756 43.18) (end 200.66 47.193756) (width 1) (layer "B.Cu") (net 3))
 (segment (start 211.249849 104.14) (end 211.94 104.14) (width 1) (layer "B.Cu") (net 3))
 (segment (start 193.98 116.84) (end 201.219138 116.84) (width 1) (layer "B.Cu") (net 3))
 (segment (start 190.21 111.47) (end 193.04 114.3) (width 1) (layer "B.Cu") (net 3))
 (segment (start 200.66 48.26) (end 198.12 50.8) (width 1) (layer "B.Cu") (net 3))
 (segment (start 205.74 101.6) (end 208.28 101.6) (width 1) (layer "B.Cu") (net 3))
 (segment (start 208.28 111.76) (end 208.28 107.816955) (width 1) (layer "B.Cu") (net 3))
 (segment (start 208.28 107.816955) (end 210.03 106.066955) (width 1) (layer "B.Cu") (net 3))
 (segment (start 218.44 111.76) (end 211.94 111.76) (width 1) (layer "B.Cu") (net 3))
 (segment (start 218.44 104.14) (end 211.94 104.14) (width 1) (layer "B.Cu") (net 3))
 (segment (start 207.79 44.870862) (end 206.099138 43.18) (width 1) (layer "B.Cu") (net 3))
 (segment (start 193.04 114.3) (end 193.04 115.9) (width 1) (layer "B.Cu") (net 3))
 (segment (start 198.12 50.8) (end 201.45 54.13) (width 1) (layer "B.Cu") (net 3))
 (segment (start 190.5 53.34) (end 190.5 50.8) (width 1) (layer "B.Cu") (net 3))
 (segment (start 206.099138 43.18) (end 204.673756 43.18) (width 1) (layer "B.Cu") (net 3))
 (segment (start 201.219138 116.84) (end 205.74 112.319138) (width 1) (layer "B.Cu") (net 3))
 (segment (start 209.4 101.6) (end 208.28 101.6) (width 1) (layer "B.Cu") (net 3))
 (segment (start 211.94 104.14) (end 209.4 101.6) (width 1) (layer "B.Cu") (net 3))
 (segment (start 206.87137 48.26) (end 207.79 47.34137) (width 1) (layer "B.Cu") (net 3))
 (segment (start 210.03 106.066955) (end 210.03 105.359849) (width 1) (layer "B.Cu") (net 3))
 (segment (start 200.66 47.193756) (end 200.66 48.26) (width 1) (layer "B.Cu") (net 3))
 (segment (start 210.03 105.359849) (end 211.249849 104.14) (width 1) (layer "B.Cu") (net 3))
 (segment (start 205.74 48.26) (end 206.87137 48.26) (width 1) (layer "B.Cu") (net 3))
 (segment (start 205.74 112.319138) (end 205.74 111.76) (width 1) (layer "B.Cu") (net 3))
 (segment (start 195.58 59.82863) (end 191.63137 55.88) (width 1) (layer "B.Cu") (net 4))
 (segment (start 187.96 91.44) (end 189.162081 91.44) (width 1) (layer "B.Cu") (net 4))
 (segment (start 191.63137 55.88) (end 190.5 55.88) (width 1) (layer "B.Cu") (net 4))
 (segment (start 189.162081 91.44) (end 195.58 85.022081) (width 1) (layer "B.Cu") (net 4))
 (segment (start 195.58 85.022081) (end 195.58 59.82863) (width 1) (layer "B.Cu") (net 4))
 (segment (start 193.774874 105.945126) (end 193.774874 98.485025) (width 1) (layer "B.Cu") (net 38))
 (segment (start 189.269849 93.98) (end 187.96 93.98) (width 1) (layer "B.Cu") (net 38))
 (segment (start 193.774874 98.485025) (end 189.269849 93.98) (width 1) (layer "B.Cu") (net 38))
 (segment (start 200.66 112.830252) (end 193.774874 105.945126) (width 1) (layer "B.Cu") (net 38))
 (segment (start 200.66 114.3) (end 200.66 112.830252) (width 1) (layer "B.Cu") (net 38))
 (segment (start 198.12 112.765126) (end 191.267437 105.912563) (width 1) (layer "B.Cu") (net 39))
 (segment (start 198.12 114.3) (end 198.12 112.765126) (width 1) (layer "B.Cu") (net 39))
 (segment (start 189.269849 96.52) (end 187.96 96.52) (width 1) (layer "B.Cu") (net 39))
 (segment (start 191.267437 105.912563) (end 191.267437 98.517588) (width 1) (layer "B.Cu") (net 39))
 (segment (start 191.267437 98.517588) (end 189.269849 96.52) (width 1) (layer "B.Cu") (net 39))
 (segment (start 195.58 112.7) (end 189.12 106.24) (width 1) (layer "B.Cu") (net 32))
 (segment (start 189.12 106.24) (end 186.317919 106.24) (width 1) (layer "B.Cu") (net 32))
 (segment (start 195.58 114.3) (end 195.58 112.7) (width 1) (layer "B.Cu") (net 32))
 (segment (start 185.42 105.342081) (end 185.42 104.14) (width 1) (layer "B.Cu") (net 32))
 (segment (start 186.317919 106.24) (end 185.42 105.342081) (width 1) (layer "B.Cu") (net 32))
 (segment (start 189.162081 88.9) (end 193.04 85.022081) (width 1) (layer "B.Cu") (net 5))
 (segment (start 187.96 88.9) (end 189.162081 88.9) (width 1) (layer "B.Cu") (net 5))
 (segment (start 193.04 59.82863) (end 191.63137 58.42) (width 1) (layer "B.Cu") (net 5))
 (segment (start 191.63137 58.42) (end 190.5 58.42) (width 1) (layer "B.Cu") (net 5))
 (segment (start 193.04 85.022081) (end 193.04 59.82863) (width 1) (layer "B.Cu") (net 5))
 (segment (start 213.421981 91.44) (end 208.28 91.44) (width 1) (layer "B.Cu") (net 23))
 (segment (start 211.94 107.26) (end 218.44 107.26) (width 1) (layer "B.Cu") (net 23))
 (segment (start 220.98 106.134213) (end 220.98 98.998019) (width 1) (layer "B.Cu") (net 23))
 (segment (start 219.854213 107.26) (end 220.98 106.134213) (width 1) (layer "B.Cu") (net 23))
 (segment (start 220.98 98.998019) (end 213.421981 91.44) (width 1) (layer "B.Cu") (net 23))
 (segment (start 218.44 107.26) (end 219.854213 107.26) (width 1) (layer "B.Cu") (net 23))
 (segment (start 211.94 96.437919) (end 211.94 99.64) (width 1) (layer "B.Cu") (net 24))
 (segment (start 209.482081 93.98) (end 211.94 96.437919) (width 1) (layer "B.Cu") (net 24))
 (segment (start 208.28 93.98) (end 209.482081 93.98) (width 1) (layer "B.Cu") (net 24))
 (segment (start 218.44 99.64) (end 211.94 99.64) (width 1) (layer "B.Cu") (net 24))
 (segment (start 181.05 104.767919) (end 184.217919 101.6) (width 1) (layer "B.Cu") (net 25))
 (segment (start 181.05 106.97) (end 181.05 104.767919) (width 1) (layer "B.Cu") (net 25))
 (segment (start 174.55 106.97) (end 181.05 106.97) (width 1) (layer "B.Cu") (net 25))
 (segment (start 184.217919 101.6) (end 185.42 101.6) (width 1) (layer "B.Cu") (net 25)))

